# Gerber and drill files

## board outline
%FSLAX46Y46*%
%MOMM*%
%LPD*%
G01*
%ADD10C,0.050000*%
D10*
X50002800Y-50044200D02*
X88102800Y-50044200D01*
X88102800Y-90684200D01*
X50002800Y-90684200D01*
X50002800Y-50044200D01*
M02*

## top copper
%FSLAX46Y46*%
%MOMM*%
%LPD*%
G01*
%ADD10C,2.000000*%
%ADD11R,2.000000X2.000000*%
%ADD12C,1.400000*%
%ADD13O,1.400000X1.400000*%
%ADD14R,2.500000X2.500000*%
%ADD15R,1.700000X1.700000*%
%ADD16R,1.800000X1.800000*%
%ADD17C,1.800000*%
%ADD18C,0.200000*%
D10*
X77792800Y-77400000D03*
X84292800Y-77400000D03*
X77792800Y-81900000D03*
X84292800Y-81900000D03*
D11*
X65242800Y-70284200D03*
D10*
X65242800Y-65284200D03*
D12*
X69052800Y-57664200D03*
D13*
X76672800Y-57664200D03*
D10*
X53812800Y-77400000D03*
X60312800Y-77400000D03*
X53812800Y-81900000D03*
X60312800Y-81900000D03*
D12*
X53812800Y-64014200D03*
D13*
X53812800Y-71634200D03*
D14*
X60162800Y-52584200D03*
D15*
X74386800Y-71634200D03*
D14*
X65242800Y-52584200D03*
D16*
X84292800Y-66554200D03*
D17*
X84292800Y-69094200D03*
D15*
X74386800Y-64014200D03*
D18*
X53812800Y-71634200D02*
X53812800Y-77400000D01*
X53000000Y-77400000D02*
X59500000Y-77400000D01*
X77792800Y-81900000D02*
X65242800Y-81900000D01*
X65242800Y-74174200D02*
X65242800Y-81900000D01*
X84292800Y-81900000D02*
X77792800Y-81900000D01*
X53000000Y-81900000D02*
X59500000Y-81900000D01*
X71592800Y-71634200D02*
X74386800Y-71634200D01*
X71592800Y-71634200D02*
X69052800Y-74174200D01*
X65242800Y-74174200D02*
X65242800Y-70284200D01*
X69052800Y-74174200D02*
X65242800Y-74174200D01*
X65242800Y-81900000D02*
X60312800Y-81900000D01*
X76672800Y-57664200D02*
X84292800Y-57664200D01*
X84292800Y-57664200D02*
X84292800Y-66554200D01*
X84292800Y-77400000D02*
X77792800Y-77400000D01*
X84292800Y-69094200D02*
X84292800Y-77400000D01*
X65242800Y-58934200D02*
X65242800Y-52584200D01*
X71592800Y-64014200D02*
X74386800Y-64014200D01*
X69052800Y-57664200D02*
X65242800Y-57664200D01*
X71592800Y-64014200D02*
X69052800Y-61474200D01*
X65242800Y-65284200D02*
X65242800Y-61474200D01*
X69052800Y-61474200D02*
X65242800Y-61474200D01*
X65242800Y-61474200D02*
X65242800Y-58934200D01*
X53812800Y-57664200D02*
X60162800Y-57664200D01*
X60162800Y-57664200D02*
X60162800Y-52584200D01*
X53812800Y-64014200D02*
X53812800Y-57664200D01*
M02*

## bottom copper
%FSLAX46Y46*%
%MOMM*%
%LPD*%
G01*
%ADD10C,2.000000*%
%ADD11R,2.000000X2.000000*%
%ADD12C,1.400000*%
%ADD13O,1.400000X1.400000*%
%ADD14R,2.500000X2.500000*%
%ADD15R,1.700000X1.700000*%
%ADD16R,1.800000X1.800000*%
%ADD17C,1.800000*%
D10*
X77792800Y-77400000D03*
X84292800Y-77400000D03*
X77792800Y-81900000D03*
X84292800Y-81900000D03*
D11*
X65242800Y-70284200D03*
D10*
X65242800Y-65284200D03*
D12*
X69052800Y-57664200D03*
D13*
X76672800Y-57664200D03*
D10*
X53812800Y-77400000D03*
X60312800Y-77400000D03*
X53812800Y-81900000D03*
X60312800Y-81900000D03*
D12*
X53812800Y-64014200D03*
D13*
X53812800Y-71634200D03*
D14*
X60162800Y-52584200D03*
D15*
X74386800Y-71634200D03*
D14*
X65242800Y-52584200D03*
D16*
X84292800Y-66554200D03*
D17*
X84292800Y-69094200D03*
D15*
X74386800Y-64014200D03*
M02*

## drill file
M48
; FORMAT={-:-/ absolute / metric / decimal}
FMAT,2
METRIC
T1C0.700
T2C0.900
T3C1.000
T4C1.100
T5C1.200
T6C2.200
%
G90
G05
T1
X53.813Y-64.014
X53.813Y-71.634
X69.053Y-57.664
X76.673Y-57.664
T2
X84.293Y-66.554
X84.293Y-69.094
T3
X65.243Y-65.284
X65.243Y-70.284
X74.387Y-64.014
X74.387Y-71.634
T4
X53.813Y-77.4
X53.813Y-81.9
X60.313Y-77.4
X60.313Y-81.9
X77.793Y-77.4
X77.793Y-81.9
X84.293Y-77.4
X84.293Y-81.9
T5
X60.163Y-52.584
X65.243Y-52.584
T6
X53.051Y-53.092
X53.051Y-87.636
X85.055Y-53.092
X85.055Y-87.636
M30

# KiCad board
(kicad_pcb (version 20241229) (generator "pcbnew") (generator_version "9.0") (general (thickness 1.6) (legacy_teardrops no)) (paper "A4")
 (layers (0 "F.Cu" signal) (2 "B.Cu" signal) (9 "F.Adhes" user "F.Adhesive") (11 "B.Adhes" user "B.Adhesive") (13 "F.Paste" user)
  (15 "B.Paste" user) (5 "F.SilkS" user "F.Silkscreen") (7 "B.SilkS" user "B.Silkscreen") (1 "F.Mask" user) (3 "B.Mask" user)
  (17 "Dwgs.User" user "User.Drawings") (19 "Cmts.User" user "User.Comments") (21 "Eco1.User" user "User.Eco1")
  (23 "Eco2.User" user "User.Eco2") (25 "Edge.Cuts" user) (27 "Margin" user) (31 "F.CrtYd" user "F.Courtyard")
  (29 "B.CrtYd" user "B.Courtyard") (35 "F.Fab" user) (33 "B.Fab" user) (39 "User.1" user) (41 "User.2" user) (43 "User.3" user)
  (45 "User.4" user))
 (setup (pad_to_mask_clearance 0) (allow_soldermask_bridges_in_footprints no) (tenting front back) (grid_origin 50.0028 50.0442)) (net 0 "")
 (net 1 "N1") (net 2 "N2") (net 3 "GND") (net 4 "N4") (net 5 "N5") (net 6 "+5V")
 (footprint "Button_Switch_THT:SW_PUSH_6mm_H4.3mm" (layer "F.Cu") (at 77.7928 77.4)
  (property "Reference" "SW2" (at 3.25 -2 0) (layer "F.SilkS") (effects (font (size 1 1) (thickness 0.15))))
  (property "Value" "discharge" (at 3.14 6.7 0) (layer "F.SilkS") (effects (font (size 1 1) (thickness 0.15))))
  (pad "1" thru_hole circle (at 0 0 90) (size 2 2) (drill 1.1) (layers "*.Cu" "*.Mask") (remove_unused_layers no) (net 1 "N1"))
  (pad "1" thru_hole circle (at 6.5 0 90) (size 2 2) (drill 1.1) (layers "*.Cu" "*.Mask") (remove_unused_layers no) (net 1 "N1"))
  (pad "2" thru_hole circle (at 0 4.5 90) (size 2 2) (drill 1.1) (layers "*.Cu" "*.Mask") (remove_unused_layers no) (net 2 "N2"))
  (pad "2" thru_hole circle (at 6.5 4.5 90) (size 2 2) (drill 1.1) (layers "*.Cu" "*.Mask") (remove_unused_layers no) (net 2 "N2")))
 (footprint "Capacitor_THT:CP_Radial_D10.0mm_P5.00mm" (layer "F.Cu") (at 65.2428 70.2842 90)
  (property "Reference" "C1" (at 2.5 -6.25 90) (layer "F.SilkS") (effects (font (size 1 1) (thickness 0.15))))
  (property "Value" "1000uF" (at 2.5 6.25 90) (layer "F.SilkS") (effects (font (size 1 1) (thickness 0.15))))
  (pad "1" thru_hole rect (at 0 0 90) (size 2 2) (drill 1) (layers "*.Cu" "*.Mask") (remove_unused_layers no) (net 2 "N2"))
  (pad "2" thru_hole circle (at 5 0 90) (size 2 2) (drill 1) (layers "*.Cu" "*.Mask") (remove_unused_layers no) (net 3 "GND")))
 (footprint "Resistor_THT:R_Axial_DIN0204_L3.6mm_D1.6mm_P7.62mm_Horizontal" (layer "F.Cu") (at 69.0528 57.6642)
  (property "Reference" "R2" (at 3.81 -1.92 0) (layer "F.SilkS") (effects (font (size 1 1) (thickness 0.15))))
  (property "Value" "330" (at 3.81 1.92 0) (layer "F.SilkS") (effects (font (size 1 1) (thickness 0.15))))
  (pad "1" thru_hole circle (at 0 0) (size 1.4 1.4) (drill 0.7) (layers "*.Cu" "*.Mask") (remove_unused_layers no) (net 3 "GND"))
  (pad "2" thru_hole oval (at 7.62 0) (size 1.4 1.4) (drill 0.7) (layers "*.Cu" "*.Mask") (remove_unused_layers no) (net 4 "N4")))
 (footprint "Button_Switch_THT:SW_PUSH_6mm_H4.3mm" (layer "F.Cu") (at 53.8128 77.4)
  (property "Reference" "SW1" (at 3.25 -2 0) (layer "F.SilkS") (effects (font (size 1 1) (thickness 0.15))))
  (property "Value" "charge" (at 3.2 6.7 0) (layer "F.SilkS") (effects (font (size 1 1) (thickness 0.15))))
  (pad "1" thru_hole circle (at 0 0 90) (size 2 2) (drill 1.1) (layers "*.Cu" "*.Mask") (remove_unused_layers no) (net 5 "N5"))
  (pad "1" thru_hole circle (at 6.5 0 90) (size 2 2) (drill 1.1) (layers "*.Cu" "*.Mask") (remove_unused_layers no) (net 5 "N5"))
  (pad "2" thru_hole circle (at 0 4.5 90) (size 2 2) (drill 1.1) (layers "*.Cu" "*.Mask") (remove_unused_layers no) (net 2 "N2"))
  (pad "2" thru_hole circle (at 6.5 4.5 90) (size 2 2) (drill 1.1) (layers "*.Cu" "*.Mask") (remove_unused_layers no) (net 2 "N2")))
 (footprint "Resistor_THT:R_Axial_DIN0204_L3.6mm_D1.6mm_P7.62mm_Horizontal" (layer "F.Cu") (at 53.8128 64.0142 -90)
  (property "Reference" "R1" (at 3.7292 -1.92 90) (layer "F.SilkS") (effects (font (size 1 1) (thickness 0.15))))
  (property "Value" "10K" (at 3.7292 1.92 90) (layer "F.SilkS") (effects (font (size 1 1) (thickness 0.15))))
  (pad "1" thru_hole circle (at 0 0 270) (size 1.4 1.4) (drill 0.7) (layers "*.Cu" "*.Mask") (remove_unused_layers no) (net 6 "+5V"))
  (pad "2" thru_hole oval (at 7.62 0 270) (size 1.4 1.4) (drill 0.7) (layers "*.Cu" "*.Mask") (remove_unused_layers no) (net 5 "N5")))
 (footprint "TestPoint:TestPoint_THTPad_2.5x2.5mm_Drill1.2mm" (layer "F.Cu") (at 60.1628 52.5842)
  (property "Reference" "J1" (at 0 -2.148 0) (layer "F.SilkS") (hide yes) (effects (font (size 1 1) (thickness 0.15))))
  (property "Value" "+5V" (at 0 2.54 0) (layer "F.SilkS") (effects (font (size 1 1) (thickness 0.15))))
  (pad "1" thru_hole rect (at 0 0) (size 2.5 2.5) (drill 1.2) (layers "*.Cu" "*.Mask") (remove_unused_layers no) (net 6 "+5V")))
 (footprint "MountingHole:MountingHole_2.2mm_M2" (layer "F.Cu") (at 85.0548 87.6362)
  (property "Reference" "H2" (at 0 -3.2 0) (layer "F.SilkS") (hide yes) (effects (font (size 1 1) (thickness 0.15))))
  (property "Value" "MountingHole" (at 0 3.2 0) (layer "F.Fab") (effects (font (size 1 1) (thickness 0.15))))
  (pad "" np_thru_hole circle (at 0 0) (size 2.2 2.2) (drill 2.2) (layers "*.Cu" "*.Mask")))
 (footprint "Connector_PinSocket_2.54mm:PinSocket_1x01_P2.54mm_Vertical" (layer "F.Cu") (at 74.3868 71.6342)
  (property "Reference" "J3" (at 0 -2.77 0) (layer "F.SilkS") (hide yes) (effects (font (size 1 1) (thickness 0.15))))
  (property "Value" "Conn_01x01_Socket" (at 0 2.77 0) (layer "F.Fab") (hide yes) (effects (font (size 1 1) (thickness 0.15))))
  (pad "1" thru_hole rect (at 0 0) (size 1.7 1.7) (drill 1) (layers "*.Cu" "*.Mask") (remove_unused_layers no) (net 2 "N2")))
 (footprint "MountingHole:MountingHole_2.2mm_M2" (layer "F.Cu") (at 53.0508 53.0922)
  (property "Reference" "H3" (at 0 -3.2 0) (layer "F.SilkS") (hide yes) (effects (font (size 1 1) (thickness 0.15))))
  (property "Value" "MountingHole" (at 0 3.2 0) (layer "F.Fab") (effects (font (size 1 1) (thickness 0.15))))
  (pad "" np_thru_hole circle (at 0 0) (size 2.2 2.2) (drill 2.2) (layers "*.Cu" "*.Mask")))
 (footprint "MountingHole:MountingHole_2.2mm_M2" (layer "F.Cu") (at 85.0548 53.0922)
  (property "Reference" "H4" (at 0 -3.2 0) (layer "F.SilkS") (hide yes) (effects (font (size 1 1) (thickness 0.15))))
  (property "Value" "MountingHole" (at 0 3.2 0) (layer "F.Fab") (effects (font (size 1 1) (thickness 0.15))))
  (pad "" np_thru_hole circle (at 0 0) (size 2.2 2.2) (drill 2.2) (layers "*.Cu" "*.Mask")))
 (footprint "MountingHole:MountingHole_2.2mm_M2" (layer "F.Cu") (at 53.0508 87.6362)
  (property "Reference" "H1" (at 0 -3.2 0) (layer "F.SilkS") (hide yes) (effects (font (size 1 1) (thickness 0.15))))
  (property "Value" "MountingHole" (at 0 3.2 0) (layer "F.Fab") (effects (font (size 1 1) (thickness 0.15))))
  (pad "" np_thru_hole circle (at 0 0) (size 2.2 2.2) (drill 2.2) (layers "*.Cu" "*.Mask")))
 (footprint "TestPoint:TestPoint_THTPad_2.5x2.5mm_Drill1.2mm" (layer "F.Cu") (at 65.2428 52.5842)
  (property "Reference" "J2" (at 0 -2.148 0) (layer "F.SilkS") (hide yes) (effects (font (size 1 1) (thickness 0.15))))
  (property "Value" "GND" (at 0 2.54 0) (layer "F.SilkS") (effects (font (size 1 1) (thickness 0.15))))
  (pad "1" thru_hole rect (at 0 0) (size 2.5 2.5) (drill 1.2) (layers "*.Cu" "*.Mask") (remove_unused_layers no) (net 3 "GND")))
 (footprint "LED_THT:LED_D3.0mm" (layer "F.Cu") (at 84.2928 66.5542 -90)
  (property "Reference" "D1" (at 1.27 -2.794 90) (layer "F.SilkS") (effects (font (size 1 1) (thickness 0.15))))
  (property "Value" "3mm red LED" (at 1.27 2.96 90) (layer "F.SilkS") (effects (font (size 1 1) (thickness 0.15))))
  (pad "1" thru_hole rect (at 0 0 270) (size 1.8 1.8) (drill 0.9) (layers "*.Cu" "*.Mask") (remove_unused_layers no) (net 4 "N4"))
  (pad "2" thru_hole circle (at 2.54 0 270) (size 1.8 1.8) (drill 0.9) (layers "*.Cu" "*.Mask") (remove_unused_layers no) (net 1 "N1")))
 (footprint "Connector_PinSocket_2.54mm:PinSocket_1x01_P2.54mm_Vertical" (layer "F.Cu") (at 74.3868 64.0142)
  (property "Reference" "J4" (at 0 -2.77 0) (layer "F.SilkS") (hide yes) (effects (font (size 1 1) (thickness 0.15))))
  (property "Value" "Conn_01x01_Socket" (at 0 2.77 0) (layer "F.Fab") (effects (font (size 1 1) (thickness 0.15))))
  (pad "1" thru_hole rect (at 0 0) (size 1.7 1.7) (drill 1) (layers "*.Cu" "*.Mask") (remove_unused_layers no) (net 3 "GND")))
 (gr_rect (start 50.0028 50.0442) (end 88.1028 90.6842) (stroke (width 0.05) (type default)) (fill no) (layer "Edge.Cuts"))
 (segment (start 53.8128 71.6342) (end 53.8128 77.4) (width 0.2) (layer "F.Cu") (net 5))
 (segment (start 53 77.4) (end 59.5 77.4) (width 0.2) (layer "F.Cu") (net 5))
 (segment (start 77.7928 81.9) (end 65.2428 81.9) (width 0.2) (layer "F.Cu") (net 2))
 (segment (start 65.2428 74.1742) (end 65.2428 81.9) (width 0.2) (layer "F.Cu") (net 2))
 (segment (start 84.2928 81.9) (end 77.7928 81.9) (width 0.2) (layer "F.Cu") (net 2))
 (segment (start 53 81.9) (end 59.5 81.9) (width 0.2) (layer "F.Cu") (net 2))
 (segment (start 71.5928 71.6342) (end 74.3868 71.6342) (width 0.2) (layer "F.Cu") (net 2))
 (segment (start 71.5928 71.6342) (end 69.0528 74.1742) (width 0.2) (layer "F.Cu") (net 2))
 (segment (start 65.2428 74.1742) (end 65.2428 70.2842) (width 0.2) (layer "F.Cu") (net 2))
 (segment (start 69.0528 74.1742) (end 65.2428 74.1742) (width 0.2) (layer "F.Cu") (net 2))
 (segment (start 65.2428 81.9) (end 60.3128 81.9) (width 0.2) (layer "F.Cu") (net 2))
 (segment (start 76.6728 57.6642) (end 84.2928 57.6642) (width 0.2) (layer "F.Cu") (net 4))
 (segment (start 84.2928 57.6642) (end 84.2928 66.5542) (width 0.2) (layer "F.Cu") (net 4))
 (segment (start 84.2928 77.4) (end 77.7928 77.4) (width 0.2) (layer "F.Cu") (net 1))
 (segment (start 84.2928 69.0942) (end 84.2928 77.4) (width 0.2) (layer "F.Cu") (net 1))
 (segment (start 65.2428 58.9342) (end 65.2428 52.5842) (width 0.2) (layer "F.Cu") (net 3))
 (segment (start 71.5928 64.0142) (end 74.3868 64.0142) (width 0.2) (layer "F.Cu") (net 3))
 (segment (start 69.0528 57.6642) (end 65.2428 57.6642) (width 0.2) (layer "F.Cu") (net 3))
 (segment (start 71.5928 64.0142) (end 69.0528 61.4742) (width 0.2) (layer "F.Cu") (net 3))
 (segment (start 65.2428 65.2842) (end 65.2428 61.4742) (width 0.2) (layer "F.Cu") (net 3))
 (segment (start 69.0528 61.4742) (end 65.2428 61.4742) (width 0.2) (layer "F.Cu") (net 3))
 (segment (start 65.2428 61.4742) (end 65.2428 58.9342) (width 0.2) (layer "F.Cu") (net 3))
 (segment (start 53.8128 57.6642) (end 60.1628 57.6642) (width 0.2) (layer "F.Cu") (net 6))
 (segment (start 60.1628 57.6642) (end 60.1628 52.5842) (width 0.2) (layer "F.Cu") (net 6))
 (segment (start 53.8128 64.0142) (end 53.8128 57.6642) (width 0.2) (layer "F.Cu") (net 6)))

